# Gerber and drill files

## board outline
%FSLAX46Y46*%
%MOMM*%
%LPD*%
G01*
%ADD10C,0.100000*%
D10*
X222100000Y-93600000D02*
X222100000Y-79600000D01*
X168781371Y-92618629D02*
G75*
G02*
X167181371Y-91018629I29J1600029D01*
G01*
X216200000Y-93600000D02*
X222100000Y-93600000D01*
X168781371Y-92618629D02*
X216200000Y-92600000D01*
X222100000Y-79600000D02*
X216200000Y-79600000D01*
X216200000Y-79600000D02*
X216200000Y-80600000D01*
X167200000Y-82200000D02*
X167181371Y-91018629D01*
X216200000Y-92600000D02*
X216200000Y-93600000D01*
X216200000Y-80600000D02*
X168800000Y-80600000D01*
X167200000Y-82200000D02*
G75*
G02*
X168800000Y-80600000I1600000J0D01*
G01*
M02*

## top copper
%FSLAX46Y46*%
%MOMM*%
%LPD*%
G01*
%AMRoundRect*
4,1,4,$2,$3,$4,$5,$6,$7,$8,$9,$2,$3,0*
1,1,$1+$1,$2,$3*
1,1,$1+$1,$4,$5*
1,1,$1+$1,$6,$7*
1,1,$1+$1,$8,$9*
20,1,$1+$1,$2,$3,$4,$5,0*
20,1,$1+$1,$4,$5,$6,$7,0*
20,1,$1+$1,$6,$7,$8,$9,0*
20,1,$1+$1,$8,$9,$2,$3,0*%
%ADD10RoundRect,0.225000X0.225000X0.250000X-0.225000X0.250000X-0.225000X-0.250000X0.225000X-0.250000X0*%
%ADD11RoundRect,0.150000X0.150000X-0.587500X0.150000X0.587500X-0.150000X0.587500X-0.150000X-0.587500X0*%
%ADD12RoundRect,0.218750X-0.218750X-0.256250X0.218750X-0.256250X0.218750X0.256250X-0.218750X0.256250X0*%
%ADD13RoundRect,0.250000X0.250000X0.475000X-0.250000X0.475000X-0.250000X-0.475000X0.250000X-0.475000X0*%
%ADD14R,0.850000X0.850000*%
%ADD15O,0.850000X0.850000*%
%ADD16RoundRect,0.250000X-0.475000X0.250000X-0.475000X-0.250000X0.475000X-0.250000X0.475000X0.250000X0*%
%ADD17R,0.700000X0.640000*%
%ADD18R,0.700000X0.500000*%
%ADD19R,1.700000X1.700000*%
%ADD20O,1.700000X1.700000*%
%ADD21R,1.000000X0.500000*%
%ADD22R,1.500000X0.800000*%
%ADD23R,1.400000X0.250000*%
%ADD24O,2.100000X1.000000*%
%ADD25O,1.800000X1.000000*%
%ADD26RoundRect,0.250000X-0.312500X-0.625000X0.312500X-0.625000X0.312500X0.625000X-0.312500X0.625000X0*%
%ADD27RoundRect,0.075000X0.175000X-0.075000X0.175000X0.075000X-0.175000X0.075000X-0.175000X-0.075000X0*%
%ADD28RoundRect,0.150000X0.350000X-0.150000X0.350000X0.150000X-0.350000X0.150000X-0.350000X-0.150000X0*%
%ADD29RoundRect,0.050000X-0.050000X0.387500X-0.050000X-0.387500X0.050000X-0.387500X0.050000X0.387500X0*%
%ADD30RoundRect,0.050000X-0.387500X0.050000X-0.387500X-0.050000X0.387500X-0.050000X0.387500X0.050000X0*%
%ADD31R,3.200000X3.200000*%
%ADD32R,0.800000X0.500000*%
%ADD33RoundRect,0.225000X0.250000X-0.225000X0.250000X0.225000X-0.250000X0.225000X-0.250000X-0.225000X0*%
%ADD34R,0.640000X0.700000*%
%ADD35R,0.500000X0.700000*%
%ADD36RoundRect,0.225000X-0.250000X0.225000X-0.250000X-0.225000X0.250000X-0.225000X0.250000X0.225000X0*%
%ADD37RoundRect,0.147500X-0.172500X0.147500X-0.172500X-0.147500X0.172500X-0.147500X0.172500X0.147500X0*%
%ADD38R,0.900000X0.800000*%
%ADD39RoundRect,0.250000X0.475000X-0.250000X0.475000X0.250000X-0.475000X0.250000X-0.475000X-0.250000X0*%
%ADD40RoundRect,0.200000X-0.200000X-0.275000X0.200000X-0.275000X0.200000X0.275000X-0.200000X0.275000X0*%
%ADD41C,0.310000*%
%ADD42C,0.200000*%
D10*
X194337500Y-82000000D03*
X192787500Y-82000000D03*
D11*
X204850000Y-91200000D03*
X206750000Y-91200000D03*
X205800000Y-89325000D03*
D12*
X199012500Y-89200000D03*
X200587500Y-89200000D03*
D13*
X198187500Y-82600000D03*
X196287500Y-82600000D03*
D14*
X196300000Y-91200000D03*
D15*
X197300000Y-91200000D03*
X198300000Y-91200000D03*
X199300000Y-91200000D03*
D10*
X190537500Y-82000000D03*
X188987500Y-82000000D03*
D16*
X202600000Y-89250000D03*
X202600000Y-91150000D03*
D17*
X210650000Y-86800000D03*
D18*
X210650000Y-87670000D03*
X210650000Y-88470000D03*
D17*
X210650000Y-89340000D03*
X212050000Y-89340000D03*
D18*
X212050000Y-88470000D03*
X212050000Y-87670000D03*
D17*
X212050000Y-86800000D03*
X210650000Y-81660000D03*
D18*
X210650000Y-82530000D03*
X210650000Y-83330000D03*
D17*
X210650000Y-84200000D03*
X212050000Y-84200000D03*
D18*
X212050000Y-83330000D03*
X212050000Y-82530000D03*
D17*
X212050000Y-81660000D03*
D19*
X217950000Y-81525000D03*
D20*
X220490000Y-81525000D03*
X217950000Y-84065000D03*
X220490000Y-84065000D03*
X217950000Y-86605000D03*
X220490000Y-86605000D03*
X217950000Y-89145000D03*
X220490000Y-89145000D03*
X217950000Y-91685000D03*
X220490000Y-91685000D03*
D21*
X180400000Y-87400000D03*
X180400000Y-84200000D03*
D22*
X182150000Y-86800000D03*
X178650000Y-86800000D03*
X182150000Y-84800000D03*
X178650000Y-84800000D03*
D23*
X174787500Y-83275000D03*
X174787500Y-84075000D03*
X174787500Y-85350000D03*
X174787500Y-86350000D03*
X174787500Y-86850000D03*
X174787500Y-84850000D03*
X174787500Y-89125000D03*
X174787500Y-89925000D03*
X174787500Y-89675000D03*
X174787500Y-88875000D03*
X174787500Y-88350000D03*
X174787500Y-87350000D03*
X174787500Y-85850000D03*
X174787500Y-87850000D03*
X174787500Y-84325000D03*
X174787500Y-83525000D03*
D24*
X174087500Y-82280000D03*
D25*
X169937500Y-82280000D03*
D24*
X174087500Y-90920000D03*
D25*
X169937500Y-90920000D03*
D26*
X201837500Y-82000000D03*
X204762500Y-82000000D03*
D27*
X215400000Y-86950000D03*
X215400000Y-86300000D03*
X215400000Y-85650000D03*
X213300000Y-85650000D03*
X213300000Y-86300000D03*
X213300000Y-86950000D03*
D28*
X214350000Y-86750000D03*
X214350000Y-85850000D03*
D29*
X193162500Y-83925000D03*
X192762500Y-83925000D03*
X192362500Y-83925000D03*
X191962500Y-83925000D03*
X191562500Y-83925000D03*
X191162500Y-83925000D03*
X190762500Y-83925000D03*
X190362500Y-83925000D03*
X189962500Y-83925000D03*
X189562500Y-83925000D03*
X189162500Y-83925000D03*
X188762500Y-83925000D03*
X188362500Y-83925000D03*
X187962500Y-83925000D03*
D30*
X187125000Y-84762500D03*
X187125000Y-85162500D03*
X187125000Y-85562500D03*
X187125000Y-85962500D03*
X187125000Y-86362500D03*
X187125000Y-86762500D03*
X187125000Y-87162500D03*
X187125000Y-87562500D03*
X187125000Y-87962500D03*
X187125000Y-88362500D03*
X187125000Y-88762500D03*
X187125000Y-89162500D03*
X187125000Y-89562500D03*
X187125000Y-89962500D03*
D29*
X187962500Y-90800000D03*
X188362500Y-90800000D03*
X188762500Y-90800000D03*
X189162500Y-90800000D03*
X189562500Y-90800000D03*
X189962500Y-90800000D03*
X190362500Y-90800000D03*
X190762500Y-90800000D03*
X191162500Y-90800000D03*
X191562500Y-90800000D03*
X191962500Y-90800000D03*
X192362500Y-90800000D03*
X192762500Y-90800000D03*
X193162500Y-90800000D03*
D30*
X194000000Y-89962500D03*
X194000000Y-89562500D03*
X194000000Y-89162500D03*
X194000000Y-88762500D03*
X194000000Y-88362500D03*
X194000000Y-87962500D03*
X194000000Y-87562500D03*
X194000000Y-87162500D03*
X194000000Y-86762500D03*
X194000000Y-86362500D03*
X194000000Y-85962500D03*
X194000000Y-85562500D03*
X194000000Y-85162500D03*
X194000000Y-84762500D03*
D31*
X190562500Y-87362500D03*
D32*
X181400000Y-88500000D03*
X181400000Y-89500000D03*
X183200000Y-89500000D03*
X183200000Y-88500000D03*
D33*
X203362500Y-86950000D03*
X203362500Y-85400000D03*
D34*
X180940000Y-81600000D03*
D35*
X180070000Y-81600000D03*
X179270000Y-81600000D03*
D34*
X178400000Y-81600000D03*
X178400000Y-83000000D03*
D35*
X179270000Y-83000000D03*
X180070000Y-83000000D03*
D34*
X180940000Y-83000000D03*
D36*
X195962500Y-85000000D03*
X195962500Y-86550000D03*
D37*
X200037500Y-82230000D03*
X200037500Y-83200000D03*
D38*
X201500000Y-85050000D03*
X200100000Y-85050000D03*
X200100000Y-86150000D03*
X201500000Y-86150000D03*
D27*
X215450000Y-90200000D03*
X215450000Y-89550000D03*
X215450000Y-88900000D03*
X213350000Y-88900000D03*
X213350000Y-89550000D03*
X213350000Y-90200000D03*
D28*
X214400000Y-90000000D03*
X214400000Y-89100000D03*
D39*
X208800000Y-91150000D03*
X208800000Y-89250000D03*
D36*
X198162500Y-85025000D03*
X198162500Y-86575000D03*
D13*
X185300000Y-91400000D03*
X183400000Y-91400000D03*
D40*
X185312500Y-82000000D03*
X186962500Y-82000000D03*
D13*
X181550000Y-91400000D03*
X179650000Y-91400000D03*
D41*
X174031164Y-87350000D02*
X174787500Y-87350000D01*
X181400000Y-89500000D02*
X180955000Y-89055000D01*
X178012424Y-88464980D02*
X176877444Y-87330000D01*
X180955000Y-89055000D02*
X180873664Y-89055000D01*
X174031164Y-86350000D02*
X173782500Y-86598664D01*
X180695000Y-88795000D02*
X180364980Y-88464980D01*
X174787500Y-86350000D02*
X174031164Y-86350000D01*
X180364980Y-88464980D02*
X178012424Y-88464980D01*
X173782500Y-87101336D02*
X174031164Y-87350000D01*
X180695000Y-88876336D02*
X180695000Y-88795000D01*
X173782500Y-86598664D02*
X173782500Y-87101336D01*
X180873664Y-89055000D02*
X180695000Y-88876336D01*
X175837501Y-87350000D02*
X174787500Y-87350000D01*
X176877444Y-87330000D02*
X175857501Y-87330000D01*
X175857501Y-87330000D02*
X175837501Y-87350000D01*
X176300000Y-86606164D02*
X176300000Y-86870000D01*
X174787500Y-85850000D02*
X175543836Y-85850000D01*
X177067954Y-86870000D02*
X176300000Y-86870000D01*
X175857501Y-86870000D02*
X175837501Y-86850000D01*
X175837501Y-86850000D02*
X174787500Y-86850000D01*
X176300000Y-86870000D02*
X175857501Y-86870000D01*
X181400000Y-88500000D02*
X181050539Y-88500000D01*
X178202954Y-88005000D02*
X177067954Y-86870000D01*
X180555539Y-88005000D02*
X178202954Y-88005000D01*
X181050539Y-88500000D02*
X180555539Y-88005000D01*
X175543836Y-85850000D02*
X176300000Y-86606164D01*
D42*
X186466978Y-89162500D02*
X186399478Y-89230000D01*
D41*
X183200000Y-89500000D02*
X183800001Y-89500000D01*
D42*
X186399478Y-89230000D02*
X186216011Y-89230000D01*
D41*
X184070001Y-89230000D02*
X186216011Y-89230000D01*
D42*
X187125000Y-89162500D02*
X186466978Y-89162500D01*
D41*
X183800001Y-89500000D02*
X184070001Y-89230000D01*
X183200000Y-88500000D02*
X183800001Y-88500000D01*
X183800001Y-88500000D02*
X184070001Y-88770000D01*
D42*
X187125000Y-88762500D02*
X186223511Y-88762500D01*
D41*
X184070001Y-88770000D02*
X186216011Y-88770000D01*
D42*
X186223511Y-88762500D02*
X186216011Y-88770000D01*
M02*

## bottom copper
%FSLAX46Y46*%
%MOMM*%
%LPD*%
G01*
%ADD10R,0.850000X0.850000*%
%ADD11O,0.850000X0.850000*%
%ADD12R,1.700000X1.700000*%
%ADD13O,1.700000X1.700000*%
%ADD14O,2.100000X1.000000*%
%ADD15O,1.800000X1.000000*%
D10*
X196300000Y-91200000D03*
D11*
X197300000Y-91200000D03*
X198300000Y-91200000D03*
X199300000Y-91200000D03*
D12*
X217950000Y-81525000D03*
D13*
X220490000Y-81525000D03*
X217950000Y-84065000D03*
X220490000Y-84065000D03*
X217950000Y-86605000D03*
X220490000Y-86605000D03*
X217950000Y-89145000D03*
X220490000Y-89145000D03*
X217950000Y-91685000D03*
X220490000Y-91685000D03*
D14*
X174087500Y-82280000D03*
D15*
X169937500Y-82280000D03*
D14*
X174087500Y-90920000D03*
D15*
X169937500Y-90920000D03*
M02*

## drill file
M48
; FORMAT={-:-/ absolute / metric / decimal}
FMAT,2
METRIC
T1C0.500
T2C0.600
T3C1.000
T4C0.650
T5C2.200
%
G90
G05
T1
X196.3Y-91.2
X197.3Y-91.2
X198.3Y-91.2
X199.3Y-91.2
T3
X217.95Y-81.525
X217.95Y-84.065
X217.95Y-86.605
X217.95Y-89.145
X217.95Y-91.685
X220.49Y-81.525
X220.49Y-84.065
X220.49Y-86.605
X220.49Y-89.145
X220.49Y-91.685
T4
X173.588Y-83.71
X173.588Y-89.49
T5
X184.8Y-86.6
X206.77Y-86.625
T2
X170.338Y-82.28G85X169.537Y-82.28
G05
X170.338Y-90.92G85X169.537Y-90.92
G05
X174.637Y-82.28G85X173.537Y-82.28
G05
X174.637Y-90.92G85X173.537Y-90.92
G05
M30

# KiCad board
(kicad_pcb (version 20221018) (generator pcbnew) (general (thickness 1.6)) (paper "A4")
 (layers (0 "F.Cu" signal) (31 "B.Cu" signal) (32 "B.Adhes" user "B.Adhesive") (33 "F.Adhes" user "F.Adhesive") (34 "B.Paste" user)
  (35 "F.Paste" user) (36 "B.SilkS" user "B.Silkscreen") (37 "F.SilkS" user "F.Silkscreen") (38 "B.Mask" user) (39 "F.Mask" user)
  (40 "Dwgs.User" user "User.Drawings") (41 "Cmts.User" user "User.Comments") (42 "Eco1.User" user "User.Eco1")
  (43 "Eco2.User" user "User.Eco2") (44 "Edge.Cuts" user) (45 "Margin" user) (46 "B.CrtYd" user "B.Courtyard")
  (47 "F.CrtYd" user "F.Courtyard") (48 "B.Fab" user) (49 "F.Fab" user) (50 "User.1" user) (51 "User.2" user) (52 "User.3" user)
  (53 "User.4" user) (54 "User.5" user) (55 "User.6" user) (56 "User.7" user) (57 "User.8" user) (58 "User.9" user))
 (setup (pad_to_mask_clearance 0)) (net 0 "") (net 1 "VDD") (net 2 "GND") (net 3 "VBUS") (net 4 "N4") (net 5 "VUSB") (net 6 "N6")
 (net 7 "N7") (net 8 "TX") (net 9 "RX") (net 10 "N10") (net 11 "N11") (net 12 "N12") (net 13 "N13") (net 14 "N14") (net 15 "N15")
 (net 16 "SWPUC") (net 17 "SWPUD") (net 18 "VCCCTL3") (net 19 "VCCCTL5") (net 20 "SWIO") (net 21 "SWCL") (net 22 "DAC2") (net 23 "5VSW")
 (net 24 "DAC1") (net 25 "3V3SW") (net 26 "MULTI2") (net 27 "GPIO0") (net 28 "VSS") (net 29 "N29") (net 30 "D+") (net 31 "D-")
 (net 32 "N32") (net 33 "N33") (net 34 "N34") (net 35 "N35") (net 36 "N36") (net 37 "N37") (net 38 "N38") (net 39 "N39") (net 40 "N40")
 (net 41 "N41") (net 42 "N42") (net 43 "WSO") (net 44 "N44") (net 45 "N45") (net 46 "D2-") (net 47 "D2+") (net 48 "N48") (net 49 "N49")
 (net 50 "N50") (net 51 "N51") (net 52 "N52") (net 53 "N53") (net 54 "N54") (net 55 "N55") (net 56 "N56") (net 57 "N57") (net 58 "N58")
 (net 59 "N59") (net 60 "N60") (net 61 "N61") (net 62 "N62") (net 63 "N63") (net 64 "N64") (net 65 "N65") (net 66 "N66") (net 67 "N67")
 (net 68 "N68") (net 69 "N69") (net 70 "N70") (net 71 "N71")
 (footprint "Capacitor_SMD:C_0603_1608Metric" (layer "F.Cu") (at 193.5625 82 180)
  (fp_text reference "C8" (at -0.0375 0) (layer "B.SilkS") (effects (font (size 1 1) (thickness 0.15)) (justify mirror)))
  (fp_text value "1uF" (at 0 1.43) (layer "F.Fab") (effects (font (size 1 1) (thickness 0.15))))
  (pad "1" smd roundrect (at -0.775 0 180) (size 0.9 0.95) (layers "F.Cu" "F.Paste" "F.Mask") (roundrect_rratio 0.25) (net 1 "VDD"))
  (pad "2" smd roundrect (at 0.775 0 180) (size 0.9 0.95) (layers "F.Cu" "F.Paste" "F.Mask") (roundrect_rratio 0.25) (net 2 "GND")))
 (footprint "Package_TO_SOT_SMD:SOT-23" (layer "F.Cu") (at 205.8 90.2625 90)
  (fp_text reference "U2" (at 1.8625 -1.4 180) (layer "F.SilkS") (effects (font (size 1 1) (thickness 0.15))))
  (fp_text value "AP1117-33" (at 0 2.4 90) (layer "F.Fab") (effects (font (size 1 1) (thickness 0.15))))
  (pad "1" smd roundrect (at -0.9375 -0.95 90) (size 1.475 0.6) (layers "F.Cu" "F.Paste" "F.Mask") (roundrect_rratio 0.25) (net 2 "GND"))
  (pad "2" smd roundrect (at -0.9375 0.95 90) (size 1.475 0.6) (layers "F.Cu" "F.Paste" "F.Mask") (roundrect_rratio 0.25) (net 1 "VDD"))
  (pad "3" smd roundrect (at 0.9375 0 90) (size 1.475 0.6) (layers "F.Cu" "F.Paste" "F.Mask") (roundrect_rratio 0.25) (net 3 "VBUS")))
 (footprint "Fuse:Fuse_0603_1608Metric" (layer "F.Cu") (at 199.8 89.2)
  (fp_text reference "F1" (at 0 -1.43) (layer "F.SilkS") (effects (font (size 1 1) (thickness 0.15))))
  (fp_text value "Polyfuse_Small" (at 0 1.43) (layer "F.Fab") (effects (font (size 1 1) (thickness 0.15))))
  (pad "1" smd roundrect (at -0.7875 0) (size 0.875 0.95) (layers "F.Cu" "F.Paste" "F.Mask") (roundrect_rratio 0.25) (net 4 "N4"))
  (pad "2" smd roundrect (at 0.7875 0) (size 0.875 0.95) (layers "F.Cu" "F.Paste" "F.Mask") (roundrect_rratio 0.25) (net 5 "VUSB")))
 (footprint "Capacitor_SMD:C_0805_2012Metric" (layer "F.Cu") (at 197.2375 82.6 180)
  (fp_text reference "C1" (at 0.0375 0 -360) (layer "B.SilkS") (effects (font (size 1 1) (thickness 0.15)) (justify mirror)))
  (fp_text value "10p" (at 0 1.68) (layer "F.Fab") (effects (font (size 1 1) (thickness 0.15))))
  (pad "1" smd roundrect (at -0.95 0 180) (size 1 1.45) (layers "F.Cu" "F.Paste" "F.Mask") (roundrect_rratio 0.25) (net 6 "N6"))
  (pad "2" smd roundrect (at 0.95 0 180) (size 1 1.45) (layers "F.Cu" "F.Paste" "F.Mask") (roundrect_rratio 0.25) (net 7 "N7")))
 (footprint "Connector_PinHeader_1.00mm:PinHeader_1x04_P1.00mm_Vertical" (layer "F.Cu") (at 196.3 91.2 90)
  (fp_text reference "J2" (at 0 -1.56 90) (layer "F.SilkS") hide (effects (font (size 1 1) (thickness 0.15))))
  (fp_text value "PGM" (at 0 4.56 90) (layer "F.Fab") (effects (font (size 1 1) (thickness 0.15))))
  (pad "1" thru_hole rect (at 0 0 90) (size 0.85 0.85) (drill 0.5) (layers "*.Cu" "*.Mask") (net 2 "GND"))
  (pad "2" thru_hole oval (at 0 1 90) (size 0.85 0.85) (drill 0.5) (layers "*.Cu" "*.Mask") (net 1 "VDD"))
  (pad "3" thru_hole oval (at 0 2 90) (size 0.85 0.85) (drill 0.5) (layers "*.Cu" "*.Mask") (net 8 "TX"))
  (pad "4" thru_hole oval (at 0 3 90) (size 0.85 0.85) (drill 0.5) (layers "*.Cu" "*.Mask") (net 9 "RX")))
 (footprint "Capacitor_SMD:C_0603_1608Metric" (layer "F.Cu") (at 189.7625 82 180)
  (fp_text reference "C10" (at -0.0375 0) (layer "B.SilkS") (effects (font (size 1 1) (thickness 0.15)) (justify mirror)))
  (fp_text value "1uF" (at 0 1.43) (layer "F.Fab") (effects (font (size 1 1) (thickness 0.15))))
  (pad "1" smd roundrect (at -0.775 0 180) (size 0.9 0.95) (layers "F.Cu" "F.Paste" "F.Mask") (roundrect_rratio 0.25) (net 1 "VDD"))
  (pad "2" smd roundrect (at 0.775 0 180) (size 0.9 0.95) (layers "F.Cu" "F.Paste" "F.Mask") (roundrect_rratio 0.25) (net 2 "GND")))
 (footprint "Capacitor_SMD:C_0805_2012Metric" (layer "F.Cu") (at 202.6 90.2 -90)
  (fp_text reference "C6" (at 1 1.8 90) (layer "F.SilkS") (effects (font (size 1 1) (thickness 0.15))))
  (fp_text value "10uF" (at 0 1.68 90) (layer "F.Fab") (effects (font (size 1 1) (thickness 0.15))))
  (pad "1" smd roundrect (at -0.95 0 270) (size 1 1.45) (layers "F.Cu" "F.Paste" "F.Mask") (roundrect_rratio 0.25) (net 3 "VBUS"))
  (pad "2" smd roundrect (at 0.95 0 270) (size 1 1.45) (layers "F.Cu" "F.Paste" "F.Mask") (roundrect_rratio 0.25) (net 2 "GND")))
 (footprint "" (layer "F.Cu") (at 184.8 86.6)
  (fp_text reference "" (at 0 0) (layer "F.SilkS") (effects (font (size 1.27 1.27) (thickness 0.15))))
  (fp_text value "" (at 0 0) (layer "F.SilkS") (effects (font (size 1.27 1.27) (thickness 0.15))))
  (pad "" np_thru_hole circle (at 0 0) (size 2.2 2.2) (drill 2.2) (layers "F&B.Cu" "*.Mask")))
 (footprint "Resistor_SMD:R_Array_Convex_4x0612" (layer "F.Cu") (at 211.35 88.07)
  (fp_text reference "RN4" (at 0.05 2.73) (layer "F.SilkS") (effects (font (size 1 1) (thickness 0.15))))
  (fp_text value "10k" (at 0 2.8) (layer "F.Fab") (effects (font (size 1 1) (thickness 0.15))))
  (pad "1" smd rect (at -0.7 -1.27) (size 0.7 0.64) (layers "F.Cu" "F.Paste" "F.Mask") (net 3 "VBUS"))
  (pad "2" smd rect (at -0.7 -0.4) (size 0.7 0.5) (layers "F.Cu" "F.Paste" "F.Mask") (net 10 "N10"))
  (pad "3" smd rect (at -0.7 0.4) (size 0.7 0.5) (layers "F.Cu" "F.Paste" "F.Mask") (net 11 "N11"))
  (pad "4" smd rect (at -0.7 1.27) (size 0.7 0.64) (layers "F.Cu" "F.Paste" "F.Mask") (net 1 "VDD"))
  (pad "5" smd rect (at 0.7 1.27) (size 0.7 0.64) (layers "F.Cu" "F.Paste" "F.Mask") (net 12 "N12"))
  (pad "6" smd rect (at 0.7 0.4) (size 0.7 0.5) (layers "F.Cu" "F.Paste" "F.Mask") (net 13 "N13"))
  (pad "7" smd rect (at 0.7 -0.4) (size 0.7 0.5) (layers "F.Cu" "F.Paste" "F.Mask") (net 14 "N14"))
  (pad "8" smd rect (at 0.7 -1.27) (size 0.7 0.64) (layers "F.Cu" "F.Paste" "F.Mask") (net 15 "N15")))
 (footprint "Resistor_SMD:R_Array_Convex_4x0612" (layer "F.Cu") (at 211.35 82.93)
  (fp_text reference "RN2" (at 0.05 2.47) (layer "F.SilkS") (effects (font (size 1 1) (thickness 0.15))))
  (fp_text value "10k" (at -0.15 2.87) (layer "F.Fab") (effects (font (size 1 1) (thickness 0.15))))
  (pad "1" smd rect (at -0.7 -1.27) (size 0.7 0.64) (layers "F.Cu" "F.Paste" "F.Mask") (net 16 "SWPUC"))
  (pad "2" smd rect (at -0.7 -0.4) (size 0.7 0.5) (layers "F.Cu" "F.Paste" "F.Mask") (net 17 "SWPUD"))
  (pad "3" smd rect (at -0.7 0.4) (size 0.7 0.5) (layers "F.Cu" "F.Paste" "F.Mask") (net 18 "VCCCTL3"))
  (pad "4" smd rect (at -0.7 1.27) (size 0.7 0.64) (layers "F.Cu" "F.Paste" "F.Mask") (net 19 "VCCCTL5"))
  (pad "5" smd rect (at 0.7 1.27) (size 0.7 0.64) (layers "F.Cu" "F.Paste" "F.Mask") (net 2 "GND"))
  (pad "6" smd rect (at 0.7 0.4) (size 0.7 0.5) (layers "F.Cu" "F.Paste" "F.Mask") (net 2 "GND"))
  (pad "7" smd rect (at 0.7 -0.4) (size 0.7 0.5) (layers "F.Cu" "F.Paste" "F.Mask") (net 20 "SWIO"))
  (pad "8" smd rect (at 0.7 -1.27) (size 0.7 0.64) (layers "F.Cu" "F.Paste" "F.Mask") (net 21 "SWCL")))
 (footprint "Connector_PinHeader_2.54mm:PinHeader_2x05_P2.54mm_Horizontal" (layer "F.Cu") (at 217.95 81.525)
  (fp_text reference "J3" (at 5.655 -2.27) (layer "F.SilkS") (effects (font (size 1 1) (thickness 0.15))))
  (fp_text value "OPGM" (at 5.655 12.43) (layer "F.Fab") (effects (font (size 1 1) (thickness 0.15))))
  (pad "1" thru_hole rect (at 0 0) (size 1.7 1.7) (drill 1) (layers "*.Cu" "*.Mask") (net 2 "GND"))
  (pad "2" thru_hole oval (at 2.54 0) (size 1.7 1.7) (drill 1) (layers "*.Cu" "*.Mask") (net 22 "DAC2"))
  (pad "3" thru_hole oval (at 0 2.54) (size 1.7 1.7) (drill 1) (layers "*.Cu" "*.Mask") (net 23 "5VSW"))
  (pad "4" thru_hole oval (at 2.54 2.54) (size 1.7 1.7) (drill 1) (layers "*.Cu" "*.Mask") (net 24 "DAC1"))
  (pad "5" thru_hole oval (at 0 5.08) (size 1.7 1.7) (drill 1) (layers "*.Cu" "*.Mask") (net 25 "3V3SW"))
  (pad "6" thru_hole oval (at 2.54 5.08) (size 1.7 1.7) (drill 1) (layers "*.Cu" "*.Mask") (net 25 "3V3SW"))
  (pad "7" thru_hole oval (at 0 7.62) (size 1.7 1.7) (drill 1) (layers "*.Cu" "*.Mask") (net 20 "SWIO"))
  (pad "8" thru_hole oval (at 2.54 7.62) (size 1.7 1.7) (drill 1) (layers "*.Cu" "*.Mask") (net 21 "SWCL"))
  (pad "9" thru_hole oval (at 0 10.16) (size 1.7 1.7) (drill 1) (layers "*.Cu" "*.Mask") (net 2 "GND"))
  (pad "10" thru_hole oval (at 2.54 10.16) (size 1.7 1.7) (drill 1) (layers "*.Cu" "*.Mask") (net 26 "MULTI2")))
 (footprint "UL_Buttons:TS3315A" (layer "F.Cu") (at 180.4 85.8 180)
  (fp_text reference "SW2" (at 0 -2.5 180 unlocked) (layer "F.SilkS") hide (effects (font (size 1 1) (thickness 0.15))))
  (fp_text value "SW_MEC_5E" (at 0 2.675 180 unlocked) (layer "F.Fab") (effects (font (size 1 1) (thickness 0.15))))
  (pad "" smd rect (at 0 -1.6 180) (size 1 0.5) (layers "F.Cu" "F.Paste" "F.Mask") (thermal_bridge_angle 45))
  (pad "" smd rect (at 0 1.6 180) (size 1 0.5) (layers "F.Cu" "F.Paste" "F.Mask") (thermal_bridge_angle 45))
  (pad "1" smd rect (at -1.75 -1 180) (size 1.5 0.8) (layers "F.Cu" "F.Paste" "F.Mask") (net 2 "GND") (thermal_bridge_angle 45))
  (pad "2" smd rect (at 1.75 -1 180) (size 1.5 0.8) (layers "F.Cu" "F.Paste" "F.Mask") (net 2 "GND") (thermal_bridge_angle 45))
  (pad "3" smd rect (at -1.75 1 180) (size 1.5 0.8) (layers "F.Cu" "F.Paste" "F.Mask") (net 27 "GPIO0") (thermal_bridge_angle 45))
  (pad "4" smd rect (at 1.75 1 180) (size 1.5 0.8) (layers "F.Cu" "F.Paste" "F.Mask") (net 27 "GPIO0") (thermal_bridge_angle 45)))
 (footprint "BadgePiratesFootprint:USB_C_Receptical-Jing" (layer "F.Cu") (at 174.0875 86.6 -90)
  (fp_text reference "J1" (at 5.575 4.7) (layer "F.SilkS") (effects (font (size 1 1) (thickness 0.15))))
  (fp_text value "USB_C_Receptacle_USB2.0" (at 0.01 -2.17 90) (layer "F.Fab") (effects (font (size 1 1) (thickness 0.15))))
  (pad "" np_thru_hole circle (at -2.89 0.5 270) (size 0.65 0.65) (drill 0.65) (layers "*.Cu" "*.Mask"))
  (pad "" np_thru_hole circle (at 2.89 0.5 270) (size 0.65 0.65) (drill 0.65) (layers "*.Cu" "*.Mask"))
  (pad "A1" smd rect (at -3.325 -0.7 270) (size 0.25 1.4) (layers "F.Cu" "F.Paste" "F.Mask") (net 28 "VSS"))
  (pad "A4" smd rect (at -2.525 -0.7 270) (size 0.25 1.4) (layers "F.Cu" "F.Paste" "F.Mask") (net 4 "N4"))
  (pad "A5" smd rect (at -1.25 -0.7 270) (size 0.25 1.4) (layers "F.Cu" "F.Paste" "F.Mask") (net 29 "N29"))
  (pad "A6" smd rect (at -0.25 -0.7 270) (size 0.25 1.4) (layers "F.Cu" "F.Paste" "F.Mask") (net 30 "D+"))
  (pad "A7" smd rect (at 0.25 -0.7 270) (size 0.25 1.4) (layers "F.Cu" "F.Paste" "F.Mask") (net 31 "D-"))
  (pad "A8" smd rect (at -1.75 -0.7 270) (size 0.25 1.4) (layers "F.Cu" "F.Paste" "F.Mask") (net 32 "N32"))
  (pad "A9" smd rect (at 2.525 -0.7 270) (size 0.25 1.4) (layers "F.Cu" "F.Paste" "F.Mask") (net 4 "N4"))
  (pad "A12" smd rect (at 3.325 -0.7 270) (size 0.25 1.4) (layers "F.Cu" "F.Paste" "F.Mask") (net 28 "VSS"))
  (pad "B1" smd rect (at 3.075 -0.7 270) (size 0.25 1.4) (layers "F.Cu" "F.Paste" "F.Mask") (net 28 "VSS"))
  (pad "B4" smd rect (at 2.275 -0.7 270) (size 0.25 1.4) (layers "F.Cu" "F.Paste" "F.Mask") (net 4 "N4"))
  (pad "B5" smd rect (at 1.75 -0.7 270) (size 0.25 1.4) (layers "F.Cu" "F.Paste" "F.Mask") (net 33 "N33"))
  (pad "B6" smd rect (at 0.75 -0.7 270) (size 0.25 1.4) (layers "F.Cu" "F.Paste" "F.Mask") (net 30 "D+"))
  (pad "B7" smd rect (at -0.75 -0.7 270) (size 0.25 1.4) (layers "F.Cu" "F.Paste" "F.Mask") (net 31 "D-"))
  (pad "B8" smd rect (at 1.25 -0.7 270) (size 0.25 1.4) (layers "F.Cu" "F.Paste" "F.Mask") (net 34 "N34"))
  (pad "B9" smd rect (at -2.275 -0.7 270) (size 0.25 1.4) (layers "F.Cu" "F.Paste" "F.Mask") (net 4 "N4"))
  (pad "B12" smd rect (at -3.075 -0.7 270) (size 0.25 1.4) (layers "F.Cu" "F.Paste" "F.Mask") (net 28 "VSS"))
  (pad "S1" thru_hole oval (at -4.32 0 270) (size 1 2.1) (drill oval 0.6 1.7) (layers "*.Cu" "*.Mask") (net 28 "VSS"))
  (pad "S1" thru_hole oval (at -4.32 4.15 270) (size 1 1.8) (drill oval 0.6 1.4) (layers "*.Cu" "*.Mask") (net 28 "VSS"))
  (pad "S1" thru_hole oval (at 4.32 0 270) (size 1 2.1) (drill oval 0.6 1.7) (layers "*.Cu" "*.Mask") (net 28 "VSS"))
  (pad "S1" thru_hole oval (at 4.32 4.15 270) (size 1 1.8) (drill oval 0.6 1.4) (layers "*.Cu" "*.Mask") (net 28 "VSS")))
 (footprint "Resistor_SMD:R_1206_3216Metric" (layer "F.Cu") (at 203.3 82)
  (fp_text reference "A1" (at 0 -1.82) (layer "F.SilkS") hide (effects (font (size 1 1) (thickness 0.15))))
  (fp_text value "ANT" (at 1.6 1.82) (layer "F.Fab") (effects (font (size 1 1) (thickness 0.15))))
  (pad "1" smd roundrect (at -1.4625 0) (size 1.125 1.75) (layers "F.Cu" "F.Paste" "F.Mask") (roundrect_rratio 0.222222) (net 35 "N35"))
  (pad "2" smd roundrect (at 1.4625 0) (size 1.125 1.75) (layers "F.Cu" "F.Paste" "F.Mask") (roundrect_rratio 0.222222) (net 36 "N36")))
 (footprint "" (layer "F.Cu") (at 206.77 86.625)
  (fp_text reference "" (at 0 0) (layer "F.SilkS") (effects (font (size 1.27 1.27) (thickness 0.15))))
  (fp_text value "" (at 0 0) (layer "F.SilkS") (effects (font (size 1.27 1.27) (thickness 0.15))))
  (pad "" np_thru_hole circle (at 0 0) (size 2.2 2.2) (drill 2.2) (layers "F&B.Cu" "*.Mask")))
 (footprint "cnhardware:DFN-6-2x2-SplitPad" (layer "F.Cu") (at 214.35 86.3 90)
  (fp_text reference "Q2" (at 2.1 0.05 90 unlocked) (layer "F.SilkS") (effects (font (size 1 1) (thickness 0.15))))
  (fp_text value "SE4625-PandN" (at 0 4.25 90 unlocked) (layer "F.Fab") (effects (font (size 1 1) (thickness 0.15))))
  (pad "1" smd roundrect (at -0.65 1.05 90) (size 0.3 0.5) (layers "F.Cu" "F.Paste" "F.Mask") (roundrect_rratio 0.25) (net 2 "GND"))
  (pad "2" smd roundrect (at 0 1.05 90) (size 0.3 0.5) (layers "F.Cu" "F.Paste" "F.Mask") (roundrect_rratio 0.25) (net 19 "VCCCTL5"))
  (pad "3" smd roundrect (at 0.65 1.05 90) (size 0.3 0.5) (layers "F.Cu" "F.Paste" "F.Mask") (roundrect_rratio 0.25) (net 23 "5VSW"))
  (pad "4" smd roundrect (at 0.65 -1.05 90) (size 0.3 0.5) (layers "F.Cu" "F.Paste" "F.Mask") (roundrect_rratio 0.25) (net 3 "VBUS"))
  (pad "5" smd roundrect (at 0 -1.05 90) (size 0.3 0.5) (layers "F.Cu" "F.Paste" "F.Mask") (roundrect_rratio 0.25) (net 15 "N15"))
  (pad "6" smd roundrect (at -0.65 -1.05 90) (size 0.3 0.5) (layers "F.Cu" "F.Paste" "F.Mask") (roundrect_rratio 0.25) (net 15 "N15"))
  (pad "7" smd roundrect (at -0.45 0 90) (size 0.6 1) (layers "F.Cu" "F.Paste" "F.Mask") (roundrect_rratio 0.25) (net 15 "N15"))
  (pad "8" smd roundrect (at 0.45 0 90) (size 0.6 1) (layers "F.Cu" "F.Paste" "F.Mask") (roundrect_rratio 0.25) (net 23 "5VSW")))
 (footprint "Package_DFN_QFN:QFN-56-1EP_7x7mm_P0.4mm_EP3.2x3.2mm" (layer "F.Cu") (at 190.5625 87.3625 -90)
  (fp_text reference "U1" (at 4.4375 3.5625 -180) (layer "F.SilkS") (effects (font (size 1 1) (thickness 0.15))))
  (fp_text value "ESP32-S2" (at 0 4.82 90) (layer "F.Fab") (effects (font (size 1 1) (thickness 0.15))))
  (pad "" smd roundrect (at -0.8 -0.8 270) (size 1.29 1.29) (layers "F.Paste") (roundrect_rratio 0.193798))
  (pad "" smd roundrect (at -0.8 0.8 270) (size 1.29 1.29) (layers "F.Paste") (roundrect_rratio 0.193798))
  (pad "" smd roundrect (at 0.8 -0.8 270) (size 1.29 1.29) (layers "F.Paste") (roundrect_rratio 0.193798))
  (pad "" smd roundrect (at 0.8 0.8 270) (size 1.29 1.29) (layers "F.Paste") (roundrect_rratio 0.193798))
  (pad "1" smd roundrect (at -3.4375 -2.6 270) (size 0.875 0.2) (layers "F.Cu" "F.Paste" "F.Mask") (roundrect_rratio 0.25) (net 1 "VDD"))
  (pad "2" smd roundrect (at -3.4375 -2.2 270) (size 0.875 0.2) (layers "F.Cu" "F.Paste" "F.Mask") (roundrect_rratio 0.25) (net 7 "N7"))
  (pad "3" smd roundrect (at -3.4375 -1.8 270) (size 0.875 0.2) (layers "F.Cu" "F.Paste" "F.Mask") (roundrect_rratio 0.25) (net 1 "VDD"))
  (pad "4" smd roundrect (at -3.4375 -1.4 270) (size 0.875 0.2) (layers "F.Cu" "F.Paste" "F.Mask") (roundrect_rratio 0.25) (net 1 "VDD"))
  (pad "5" smd roundrect (at -3.4375 -1 270) (size 0.875 0.2) (layers "F.Cu" "F.Paste" "F.Mask") (roundrect_rratio 0.25) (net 27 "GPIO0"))
  (pad "6" smd roundrect (at -3.4375 -0.6 270) (size 0.875 0.2) (layers "F.Cu" "F.Paste" "F.Mask") (roundrect_rratio 0.25) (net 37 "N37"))
  (pad "7" smd roundrect (at -3.4375 -0.2 270) (size 0.875 0.2) (layers "F.Cu" "F.Paste" "F.Mask") (roundrect_rratio 0.25) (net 26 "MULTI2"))
  (pad "8" smd roundrect (at -3.4375 0.2 270) (size 0.875 0.2) (layers "F.Cu" "F.Paste" "F.Mask") (roundrect_rratio 0.25) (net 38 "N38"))
  (pad "9" smd roundrect (at -3.4375 0.6 270) (size 0.875 0.2) (layers "F.Cu" "F.Paste" "F.Mask") (roundrect_rratio 0.25) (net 21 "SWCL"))
  (pad "10" smd roundrect (at -3.4375 1 270) (size 0.875 0.2) (layers "F.Cu" "F.Paste" "F.Mask") (roundrect_rratio 0.25) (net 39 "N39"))
  (pad "11" smd roundrect (at -3.4375 1.4 270) (size 0.875 0.2) (layers "F.Cu" "F.Paste" "F.Mask") (roundrect_rratio 0.25) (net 20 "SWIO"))
  (pad "12" smd roundrect (at -3.4375 1.8 270) (size 0.875 0.2) (layers "F.Cu" "F.Paste" "F.Mask") (roundrect_rratio 0.25) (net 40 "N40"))
  (pad "13" smd roundrect (at -3.4375 2.2 270) (size 0.875 0.2) (layers "F.Cu" "F.Paste" "F.Mask") (roundrect_rratio 0.25) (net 16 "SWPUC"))
  (pad "14" smd roundrect (at -3.4375 2.6 270) (size 0.875 0.2) (layers "F.Cu" "F.Paste" "F.Mask") (roundrect_rratio 0.25) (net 17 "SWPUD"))
  (pad "15" smd roundrect (at -2.6 3.4375 270) (size 0.2 0.875) (layers "F.Cu" "F.Paste" "F.Mask") (roundrect_rratio 0.25) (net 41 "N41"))
  (pad "16" smd roundrect (at -2.2 3.4375 270) (size 0.2 0.875) (layers "F.Cu" "F.Paste" "F.Mask") (roundrect_rratio 0.25)
   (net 18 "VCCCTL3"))
  (pad "17" smd roundrect (at -1.8 3.4375 270) (size 0.2 0.875) (layers "F.Cu" "F.Paste" "F.Mask") (roundrect_rratio 0.25)
   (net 19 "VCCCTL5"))
  (pad "18" smd roundrect (at -1.4 3.4375 270) (size 0.2 0.875) (layers "F.Cu" "F.Paste" "F.Mask") (roundrect_rratio 0.25) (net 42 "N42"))
  (pad "19" smd roundrect (at -1 3.4375 270) (size 0.2 0.875) (layers "F.Cu" "F.Paste" "F.Mask") (roundrect_rratio 0.25) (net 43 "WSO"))
  (pad "20" smd roundrect (at -0.6 3.4375 270) (size 0.2 0.875) (layers "F.Cu" "F.Paste" "F.Mask") (roundrect_rratio 0.25) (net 1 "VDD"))
  (pad "21" smd roundrect (at -0.2 3.4375 270) (size 0.2 0.875) (layers "F.Cu" "F.Paste" "F.Mask") (roundrect_rratio 0.25) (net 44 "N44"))
  (pad "22" smd roundrect (at 0.2 3.4375 270) (size 0.2 0.875) (layers "F.Cu" "F.Paste" "F.Mask") (roundrect_rratio 0.25) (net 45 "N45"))
  (pad "23" smd roundrect (at 0.6 3.4375 270) (size 0.2 0.875) (layers "F.Cu" "F.Paste" "F.Mask") (roundrect_rratio 0.25) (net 24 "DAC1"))
  (pad "24" smd roundrect (at 1 3.4375 270) (size 0.2 0.875) (layers "F.Cu" "F.Paste" "F.Mask") (roundrect_rratio 0.25) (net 22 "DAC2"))
  (pad "25" smd roundrect (at 1.4 3.4375 270) (size 0.2 0.875) (layers "F.Cu" "F.Paste" "F.Mask") (roundrect_rratio 0.25) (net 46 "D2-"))
  (pad "26" smd roundrect (at 1.8 3.4375 270) (size 0.2 0.875) (layers "F.Cu" "F.Paste" "F.Mask") (roundrect_rratio 0.25) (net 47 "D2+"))
  (pad "27" smd roundrect (at 2.2 3.4375 270) (size 0.2 0.875) (layers "F.Cu" "F.Paste" "F.Mask") (roundrect_rratio 0.25) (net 1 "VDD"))
  (pad "28" smd roundrect (at 2.6 3.4375 270) (size 0.2 0.875) (layers "F.Cu" "F.Paste" "F.Mask") (roundrect_rratio 0.25) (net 2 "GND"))
  (pad "29" smd roundrect (at 3.4375 2.6 270) (size 0.875 0.2) (layers "F.Cu" "F.Paste" "F.Mask") (roundrect_rratio 0.25) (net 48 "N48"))
  (pad "30" smd roundrect (at 3.4375 2.2 270) (size 0.875 0.2) (layers "F.Cu" "F.Paste" "F.Mask") (roundrect_rratio 0.25) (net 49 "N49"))
  (pad "31" smd roundrect (at 3.4375 1.8 270) (size 0.875 0.2) (layers "F.Cu" "F.Paste" "F.Mask") (roundrect_rratio 0.25) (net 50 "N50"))
  (pad "32" smd roundrect (at 3.4375 1.4 270) (size 0.875 0.2) (layers "F.Cu" "F.Paste" "F.Mask") (roundrect_rratio 0.25) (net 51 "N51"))
  (pad "33" smd roundrect (at 3.4375 1 270) (size 0.875 0.2) (layers "F.Cu" "F.Paste" "F.Mask") (roundrect_rratio 0.25) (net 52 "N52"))
  (pad "34" smd roundrect (at 3.4375 0.6 270) (size 0.875 0.2) (layers "F.Cu" "F.Paste" "F.Mask") (roundrect_rratio 0.25) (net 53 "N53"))
  (pad "35" smd roundrect (at 3.4375 0.2 270) (size 0.875 0.2) (layers "F.Cu" "F.Paste" "F.Mask") (roundrect_rratio 0.25) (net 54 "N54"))
  (pad "36" smd roundrect (at 3.4375 -0.2 270) (size 0.875 0.2) (layers "F.Cu" "F.Paste" "F.Mask") (roundrect_rratio 0.25) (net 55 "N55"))
  (pad "37" smd roundrect (at 3.4375 -0.6 270) (size 0.875 0.2) (layers "F.Cu" "F.Paste" "F.Mask") (roundrect_rratio 0.25) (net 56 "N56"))
  (pad "38" smd roundrect (at 3.4375 -1 270) (size 0.875 0.2) (layers "F.Cu" "F.Paste" "F.Mask") (roundrect_rratio 0.25) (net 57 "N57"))
  (pad "39" smd roundrect (at 3.4375 -1.4 270) (size 0.875 0.2) (layers "F.Cu" "F.Paste" "F.Mask") (roundrect_rratio 0.25) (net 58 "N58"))
  (pad "40" smd roundrect (at 3.4375 -1.8 270) (size 0.875 0.2) (layers "F.Cu" "F.Paste" "F.Mask") (roundrect_rratio 0.25) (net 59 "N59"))
  (pad "41" smd roundrect (at 3.4375 -2.2 270) (size 0.875 0.2) (layers "F.Cu" "F.Paste" "F.Mask") (roundrect_rratio 0.25) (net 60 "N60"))
  (pad "42" smd roundrect (at 3.4375 -2.6 270) (size 0.875 0.2) (layers "F.Cu" "F.Paste" "F.Mask") (roundrect_rratio 0.25) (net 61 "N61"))
  (pad "43" smd roundrect (at 2.6 -3.4375 270) (size 0.2 0.875) (layers "F.Cu" "F.Paste" "F.Mask") (roundrect_rratio 0.25) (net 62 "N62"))
  (pad "44" smd roundrect (at 2.2 -3.4375 270) (size 0.2 0.875) (layers "F.Cu" "F.Paste" "F.Mask") (roundrect_rratio 0.25) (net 2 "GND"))
  (pad "45" smd roundrect (at 1.8 -3.4375 270) (size 0.2 0.875) (layers "F.Cu" "F.Paste" "F.Mask") (roundrect_rratio 0.25) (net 1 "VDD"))
  (pad "46" smd roundrect (at 1.4 -3.4375 270) (size 0.2 0.875) (layers "F.Cu" "F.Paste" "F.Mask") (roundrect_rratio 0.25) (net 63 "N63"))
  (pad "47" smd roundrect (at 1 -3.4375 270) (size 0.2 0.875) (layers "F.Cu" "F.Paste" "F.Mask") (roundrect_rratio 0.25) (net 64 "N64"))
  (pad "48" smd roundrect (at 0.6 -3.4375 270) (size 0.2 0.875) (layers "F.Cu" "F.Paste" "F.Mask") (roundrect_rratio 0.25) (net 8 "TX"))
  (pad "49" smd roundrect (at 0.2 -3.4375 270) (size 0.2 0.875) (layers "F.Cu" "F.Paste" "F.Mask") (roundrect_rratio 0.25) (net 9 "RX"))
  (pad "50" smd roundrect (at -0.2 -3.4375 270) (size 0.2 0.875) (layers "F.Cu" "F.Paste" "F.Mask") (roundrect_rratio 0.25) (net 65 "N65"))
  (pad "51" smd roundrect (at -0.6 -3.4375 270) (size 0.2 0.875) (layers "F.Cu" "F.Paste" "F.Mask") (roundrect_rratio 0.25) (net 1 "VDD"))
  (pad "52" smd roundrect (at -1 -3.4375 270) (size 0.2 0.875) (layers "F.Cu" "F.Paste" "F.Mask") (roundrect_rratio 0.25) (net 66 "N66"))
  (pad "53" smd roundrect (at -1.4 -3.4375 270) (size 0.2 0.875) (layers "F.Cu" "F.Paste" "F.Mask") (roundrect_rratio 0.25) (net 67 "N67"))
  (pad "54" smd roundrect (at -1.8 -3.4375 270) (size 0.2 0.875) (layers "F.Cu" "F.Paste" "F.Mask") (roundrect_rratio 0.25) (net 1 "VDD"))
  (pad "55" smd roundrect (at -2.2 -3.4375 270) (size 0.2 0.875) (layers "F.Cu" "F.Paste" "F.Mask") (roundrect_rratio 0.25) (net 2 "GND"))
  (pad "56" smd roundrect (at -2.6 -3.4375 270) (size 0.2 0.875) (layers "F.Cu" "F.Paste" "F.Mask") (roundrect_rratio 0.25) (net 1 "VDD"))
  (pad "57" smd rect (at 0 0 270) (size 3.2 3.2) (layers "F.Cu" "F.Mask") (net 2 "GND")))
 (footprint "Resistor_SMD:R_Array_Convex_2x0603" (layer "F.Cu") (at 182.3 89)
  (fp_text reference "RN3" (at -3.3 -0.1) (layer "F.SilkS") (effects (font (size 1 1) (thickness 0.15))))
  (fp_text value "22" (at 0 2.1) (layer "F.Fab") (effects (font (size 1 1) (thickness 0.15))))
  (pad "1" smd rect (at -0.9 -0.5) (size 0.8 0.5) (layers "F.Cu" "F.Paste" "F.Mask") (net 31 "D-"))
  (pad "2" smd rect (at -0.9 0.5) (size 0.8 0.5) (layers "F.Cu" "F.Paste" "F.Mask") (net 30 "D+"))
  (pad "3" smd rect (at 0.9 0.5) (size 0.8 0.5) (layers "F.Cu" "F.Paste" "F.Mask") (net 47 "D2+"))
  (pad "4" smd rect (at 0.9 -0.5) (size 0.8 0.5) (layers "F.Cu" "F.Paste" "F.Mask") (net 46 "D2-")))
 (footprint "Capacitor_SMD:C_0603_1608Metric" (layer "F.Cu") (at 203.3625 86.175 90)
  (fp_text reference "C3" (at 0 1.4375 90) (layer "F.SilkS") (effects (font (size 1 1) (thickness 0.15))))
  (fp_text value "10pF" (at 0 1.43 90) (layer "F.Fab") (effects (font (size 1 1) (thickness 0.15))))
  (pad "1" smd roundrect (at -0.775 0 90) (size 0.9 0.95) (layers "F.Cu" "F.Paste" "F.Mask") (roundrect_rratio 0.25) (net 2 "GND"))
  (pad "2" smd roundrect (at 0.775 0 90) (size 0.9 0.95) (layers "F.Cu" "F.Paste" "F.Mask") (roundrect_rratio 0.25) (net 67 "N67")))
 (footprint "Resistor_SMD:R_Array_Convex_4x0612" (layer "F.Cu") (at 179.67 82.3 -90)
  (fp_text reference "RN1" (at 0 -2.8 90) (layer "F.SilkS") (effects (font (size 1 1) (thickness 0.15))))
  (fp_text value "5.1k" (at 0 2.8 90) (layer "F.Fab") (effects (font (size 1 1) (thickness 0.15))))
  (pad "1" smd rect (at -0.7 -1.27 270) (size 0.7 0.64) (layers "F.Cu" "F.Paste" "F.Mask") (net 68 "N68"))
  (pad "2" smd rect (at -0.7 -0.4 270) (size 0.7 0.5) (layers "F.Cu" "F.Paste" "F.Mask") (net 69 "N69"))
  (pad "3" smd rect (at -0.7 0.4 270) (size 0.7 0.5) (layers "F.Cu" "F.Paste" "F.Mask") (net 28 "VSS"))
  (pad "4" smd rect (at -0.7 1.27 270) (size 0.7 0.64) (layers "F.Cu" "F.Paste" "F.Mask") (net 28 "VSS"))
  (pad "5" smd rect (at 0.7 1.27 270) (size 0.7 0.64) (layers "F.Cu" "F.Paste" "F.Mask") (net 33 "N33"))
  (pad "6" smd rect (at 0.7 0.4 270) (size 0.7 0.5) (layers "F.Cu" "F.Paste" "F.Mask") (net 29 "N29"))
  (pad "7" smd rect (at 0.7 -0.4 270) (size 0.7 0.5) (layers "F.Cu" "F.Paste" "F.Mask") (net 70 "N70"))
  (pad "8" smd rect (at 0.7 -1.27 270) (size 0.7 0.64) (layers "F.Cu" "F.Paste" "F.Mask") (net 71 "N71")))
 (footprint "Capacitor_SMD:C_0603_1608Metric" (layer "F.Cu") (at 195.9625 85.775 -90)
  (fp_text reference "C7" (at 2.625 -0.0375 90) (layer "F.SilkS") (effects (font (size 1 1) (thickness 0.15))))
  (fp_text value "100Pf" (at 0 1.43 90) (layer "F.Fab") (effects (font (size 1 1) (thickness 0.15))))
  (pad "1" smd roundrect (at -0.775 0 270) (size 0.9 0.95) (layers "F.Cu" "F.Paste" "F.Mask") (roundrect_rratio 0.25) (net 1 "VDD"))
  (pad "2" smd roundrect (at 0.775 0 270) (size 0.9 0.95) (layers "F.Cu" "F.Paste" "F.Mask") (roundrect_rratio 0.25) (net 2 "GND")))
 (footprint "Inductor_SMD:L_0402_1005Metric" (layer "F.Cu") (at 200.0375 82.715 -90)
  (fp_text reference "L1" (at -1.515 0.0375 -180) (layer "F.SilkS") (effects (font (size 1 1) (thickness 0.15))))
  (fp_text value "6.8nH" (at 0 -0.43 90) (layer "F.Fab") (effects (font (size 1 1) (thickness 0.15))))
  (pad "1" smd roundrect (at -0.485 0 270) (size 0.59 0.64) (layers "F.Cu" "F.Paste" "F.Mask") (roundrect_rratio 0.25) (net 35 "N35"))
  (pad "2" smd roundrect (at 0.485 0 270) (size 0.59 0.64) (layers "F.Cu" "F.Paste" "F.Mask") (roundrect_rratio 0.25) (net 6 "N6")))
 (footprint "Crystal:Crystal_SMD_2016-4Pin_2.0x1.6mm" (layer "F.Cu") (at 200.8 85.6 180)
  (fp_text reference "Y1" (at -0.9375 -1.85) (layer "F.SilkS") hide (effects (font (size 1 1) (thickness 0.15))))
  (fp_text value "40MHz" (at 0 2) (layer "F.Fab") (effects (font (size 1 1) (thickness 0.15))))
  (pad "1" smd rect (at -0.7 0.55 180) (size 0.9 0.8) (layers "F.Cu" "F.Paste" "F.Mask") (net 67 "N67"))
  (pad "2" smd rect (at 0.7 0.55 180) (size 0.9 0.8) (layers "F.Cu" "F.Paste" "F.Mask") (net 2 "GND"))
  (pad "3" smd rect (at 0.7 -0.55 180) (size 0.9 0.8) (layers "F.Cu" "F.Paste" "F.Mask") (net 66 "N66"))
  (pad "4" smd rect (at -0.7 -0.55 180) (size 0.9 0.8) (layers "F.Cu" "F.Paste" "F.Mask") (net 2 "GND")))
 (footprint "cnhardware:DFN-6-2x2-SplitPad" (layer "F.Cu") (at 214.4 89.55 90)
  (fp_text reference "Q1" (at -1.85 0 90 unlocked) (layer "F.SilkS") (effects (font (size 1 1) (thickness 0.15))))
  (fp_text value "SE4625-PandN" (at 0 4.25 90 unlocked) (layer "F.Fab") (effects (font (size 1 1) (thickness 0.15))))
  (pad "1" smd roundrect (at -0.65 1.05 90) (size 0.3 0.5) (layers "F.Cu" "F.Paste" "F.Mask") (roundrect_rratio 0.25) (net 2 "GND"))
  (pad "2" smd roundrect (at 0 1.05 90) (size 0.3 0.5) (layers "F.Cu" "F.Paste" "F.Mask") (roundrect_rratio 0.25) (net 18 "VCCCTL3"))
  (pad "3" smd roundrect (at 0.65 1.05 90) (size 0.3 0.5) (layers "F.Cu" "F.Paste" "F.Mask") (roundrect_rratio 0.25) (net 25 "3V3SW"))
  (pad "4" smd roundrect (at 0.65 -1.05 90) (size 0.3 0.5) (layers "F.Cu" "F.Paste" "F.Mask") (roundrect_rratio 0.25) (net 1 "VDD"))
  (pad "5" smd roundrect (at 0 -1.05 90) (size 0.3 0.5) (layers "F.Cu" "F.Paste" "F.Mask") (roundrect_rratio 0.25) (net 12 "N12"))
  (pad "6" smd roundrect (at -0.65 -1.05 90) (size 0.3 0.5) (layers "F.Cu" "F.Paste" "F.Mask") (roundrect_rratio 0.25) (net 12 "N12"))
  (pad "7" smd roundrect (at -0.45 0 90) (size 0.6 1) (layers "F.Cu" "F.Paste" "F.Mask") (roundrect_rratio 0.25) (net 12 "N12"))
  (pad "8" smd roundrect (at 0.45 0 90) (size 0.6 1) (layers "F.Cu" "F.Paste" "F.Mask") (roundrect_rratio 0.25) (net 25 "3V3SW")))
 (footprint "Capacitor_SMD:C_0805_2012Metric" (layer "F.Cu") (at 208.8 90.2 90)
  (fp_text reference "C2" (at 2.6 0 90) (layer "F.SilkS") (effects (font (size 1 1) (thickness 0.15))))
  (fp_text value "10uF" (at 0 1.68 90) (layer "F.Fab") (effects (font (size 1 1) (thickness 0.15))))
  (pad "1" smd roundrect (at -0.95 0 90) (size 1 1.45) (layers "F.Cu" "F.Paste" "F.Mask") (roundrect_rratio 0.25) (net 1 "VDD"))
  (pad "2" smd roundrect (at 0.95 0 90) (size 1 1.45) (layers "F.Cu" "F.Paste" "F.Mask") (roundrect_rratio 0.25) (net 2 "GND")))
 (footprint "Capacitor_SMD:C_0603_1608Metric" (layer "F.Cu") (at 198.1625 85.8 -90)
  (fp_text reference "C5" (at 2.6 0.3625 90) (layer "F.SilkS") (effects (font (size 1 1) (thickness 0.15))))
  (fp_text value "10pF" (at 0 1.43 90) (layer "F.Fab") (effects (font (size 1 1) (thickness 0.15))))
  (pad "1" smd roundrect (at -0.775 0 270) (size 0.9 0.95) (layers "F.Cu" "F.Paste" "F.Mask") (roundrect_rratio 0.25) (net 2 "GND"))
  (pad "2" smd roundrect (at 0.775 0 270) (size 0.9 0.95) (layers "F.Cu" "F.Paste" "F.Mask") (roundrect_rratio 0.25) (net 66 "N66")))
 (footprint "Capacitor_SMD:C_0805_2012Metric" (layer "F.Cu") (at 184.35 91.4 180)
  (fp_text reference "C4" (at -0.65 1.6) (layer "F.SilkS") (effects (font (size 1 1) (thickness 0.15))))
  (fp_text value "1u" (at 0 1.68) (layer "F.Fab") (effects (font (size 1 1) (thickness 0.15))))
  (pad "1" smd roundrect (at -0.95 0 180) (size 1 1.45) (layers "F.Cu" "F.Paste" "F.Mask") (roundrect_rratio 0.25) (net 49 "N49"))
  (pad "2" smd roundrect (at 0.95 0 180) (size 1 1.45) (layers "F.Cu" "F.Paste" "F.Mask") (roundrect_rratio 0.25) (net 2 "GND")))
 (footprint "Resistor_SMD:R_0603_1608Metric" (layer "F.Cu") (at 186.1375 82)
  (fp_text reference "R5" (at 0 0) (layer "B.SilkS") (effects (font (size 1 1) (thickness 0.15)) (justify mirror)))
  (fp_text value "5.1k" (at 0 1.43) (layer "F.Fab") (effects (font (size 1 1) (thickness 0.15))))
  (pad "1" smd roundrect (at -0.825 0) (size 0.8 0.95) (layers "F.Cu" "F.Paste" "F.Mask") (roundrect_rratio 0.25) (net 1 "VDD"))
  (pad "2" smd roundrect (at 0.825 0) (size 0.8 0.95) (layers "F.Cu" "F.Paste" "F.Mask") (roundrect_rratio 0.25) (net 27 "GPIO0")))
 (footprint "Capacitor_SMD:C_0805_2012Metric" (layer "F.Cu") (at 180.6 91.4 180)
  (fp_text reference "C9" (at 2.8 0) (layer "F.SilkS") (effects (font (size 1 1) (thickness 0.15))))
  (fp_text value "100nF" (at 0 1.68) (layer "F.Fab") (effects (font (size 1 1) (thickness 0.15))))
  (pad "1" smd roundrect (at -0.95 0 180) (size 1 1.45) (layers "F.Cu" "F.Paste" "F.Mask") (roundrect_rratio 0.25) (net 1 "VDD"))
  (pad "2" smd roundrect (at 0.95 0 180) (size 1 1.45) (layers "F.Cu" "F.Paste" "F.Mask") (roundrect_rratio 0.25) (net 2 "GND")))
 (gr_line (start 222.1 93.6) (end 222.1 79.6) (stroke (width 0.1) (type default)) (layer "Edge.Cuts"))
 (gr_arc (start 168.781371 92.618629) (mid 167.650009 92.149991) (end 167.181371 91.018629) (stroke (width 0.1) (type default))
  (layer "Edge.Cuts"))
 (gr_line (start 216.2 93.6) (end 222.1 93.6) (stroke (width 0.1) (type default)) (layer "Edge.Cuts"))
 (gr_line (start 168.781371 92.618629) (end 216.2 92.6) (stroke (width 0.1) (type default)) (layer "Edge.Cuts"))
 (gr_line (start 222.1 79.6) (end 216.2 79.6) (stroke (width 0.1) (type default)) (layer "Edge.Cuts"))
 (gr_line (start 216.2 79.6) (end 216.2 80.6) (stroke (width 0.1) (type default)) (layer "Edge.Cuts"))
 (gr_line (start 167.2 82.2) (end 167.181371 91.018629) (stroke (width 0.1) (type default)) (layer "Edge.Cuts"))
 (gr_line (start 216.2 92.6) (end 216.2 93.6) (stroke (width 0.1) (type default)) (layer "Edge.Cuts"))
 (gr_line (start 216.2 80.6) (end 168.8 80.6) (stroke (width 0.1) (type default)) (layer "Edge.Cuts"))
 (gr_arc (start 167.2 82.2) (mid 167.668629 81.068629) (end 168.8 80.6) (stroke (width 0.1) (type default)) (layer "Edge.Cuts"))
 (segment (start 174.031164 87.35) (end 174.7875 87.35) (width 0.31) (layer "F.Cu") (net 30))
 (segment (start 181.4 89.5) (end 180.955 89.055) (width 0.31) (layer "F.Cu") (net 30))
 (segment (start 178.012424 88.46498) (end 176.877444 87.33) (width 0.31) (layer "F.Cu") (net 30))
 (segment (start 180.955 89.055) (end 180.873664 89.055) (width 0.31) (layer "F.Cu") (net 30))
 (segment (start 174.031164 86.35) (end 173.7825 86.598664) (width 0.31) (layer "F.Cu") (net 30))
 (segment (start 180.695 88.795) (end 180.36498 88.46498) (width 0.31) (layer "F.Cu") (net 30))
 (segment (start 174.7875 86.35) (end 174.031164 86.35) (width 0.31) (layer "F.Cu") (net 30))
 (segment (start 180.36498 88.46498) (end 178.012424 88.46498) (width 0.31) (layer "F.Cu") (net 30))
 (segment (start 173.7825 87.101336) (end 174.031164 87.35) (width 0.31) (layer "F.Cu") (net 30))
 (segment (start 180.695 88.876336) (end 180.695 88.795) (width 0.31) (layer "F.Cu") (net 30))
 (segment (start 173.7825 86.598664) (end 173.7825 87.101336) (width 0.31) (layer "F.Cu") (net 30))
 (segment (start 180.873664 89.055) (end 180.695 88.876336) (width 0.31) (layer "F.Cu") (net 30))
 (segment (start 175.837501 87.35) (end 174.7875 87.35) (width 0.31) (layer "F.Cu") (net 30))
 (segment (start 176.877444 87.33) (end 175.857501 87.33) (width 0.31) (layer "F.Cu") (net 30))
 (segment (start 175.857501 87.33) (end 175.837501 87.35) (width 0.31) (layer "F.Cu") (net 30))
 (segment (start 176.3 86.606164) (end 176.3 86.87) (width 0.31) (layer "F.Cu") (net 31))
 (segment (start 174.7875 85.85) (end 175.543836 85.85) (width 0.31) (layer "F.Cu") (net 31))
 (segment (start 177.067954 86.87) (end 176.3 86.87) (width 0.31) (layer "F.Cu") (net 31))
 (segment (start 175.857501 86.87) (end 175.837501 86.85) (width 0.31) (layer "F.Cu") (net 31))
 (segment (start 175.837501 86.85) (end 174.7875 86.85) (width 0.31) (layer "F.Cu") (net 31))
 (segment (start 176.3 86.87) (end 175.857501 86.87) (width 0.31) (layer "F.Cu") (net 31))
 (segment (start 181.4 88.5) (end 181.050539 88.5) (width 0.31) (layer "F.Cu") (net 31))
 (segment (start 178.202954 88.005) (end 177.067954 86.87) (width 0.31) (layer "F.Cu") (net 31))
 (segment (start 180.555539 88.005) (end 178.202954 88.005) (width 0.31) (layer "F.Cu") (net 31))
 (segment (start 181.050539 88.5) (end 180.555539 88.005) (width 0.31) (layer "F.Cu") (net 31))
 (segment (start 175.543836 85.85) (end 176.3 86.606164) (width 0.31) (layer "F.Cu") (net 31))
 (segment (start 186.466978 89.1625) (end 186.399478 89.23) (width 0.2) (layer "F.Cu") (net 47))
 (segment (start 183.2 89.5) (end 183.800001 89.5) (width 0.31) (layer "F.Cu") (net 47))
 (segment (start 186.399478 89.23) (end 186.216011 89.23) (width 0.2) (layer "F.Cu") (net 47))
 (segment (start 184.070001 89.23) (end 186.216011 89.23) (width 0.31) (layer "F.Cu") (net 47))
 (segment (start 187.125 89.1625) (end 186.466978 89.1625) (width 0.2) (layer "F.Cu") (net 47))
 (segment (start 183.800001 89.5) (end 184.070001 89.23) (width 0.31) (layer "F.Cu") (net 47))
 (segment (start 183.2 88.5) (end 183.800001 88.5) (width 0.31) (layer "F.Cu") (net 46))
 (segment (start 183.800001 88.5) (end 184.070001 88.77) (width 0.31) (layer "F.Cu") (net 46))
 (segment (start 187.125 88.7625) (end 186.223511 88.7625) (width 0.2) (layer "F.Cu") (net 46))
 (segment (start 184.070001 88.77) (end 186.216011 88.77) (width 0.31) (layer "F.Cu") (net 46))
 (segment (start 186.223511 88.7625) (end 186.216011 88.77) (width 0.2) (layer "F.Cu") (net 46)))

